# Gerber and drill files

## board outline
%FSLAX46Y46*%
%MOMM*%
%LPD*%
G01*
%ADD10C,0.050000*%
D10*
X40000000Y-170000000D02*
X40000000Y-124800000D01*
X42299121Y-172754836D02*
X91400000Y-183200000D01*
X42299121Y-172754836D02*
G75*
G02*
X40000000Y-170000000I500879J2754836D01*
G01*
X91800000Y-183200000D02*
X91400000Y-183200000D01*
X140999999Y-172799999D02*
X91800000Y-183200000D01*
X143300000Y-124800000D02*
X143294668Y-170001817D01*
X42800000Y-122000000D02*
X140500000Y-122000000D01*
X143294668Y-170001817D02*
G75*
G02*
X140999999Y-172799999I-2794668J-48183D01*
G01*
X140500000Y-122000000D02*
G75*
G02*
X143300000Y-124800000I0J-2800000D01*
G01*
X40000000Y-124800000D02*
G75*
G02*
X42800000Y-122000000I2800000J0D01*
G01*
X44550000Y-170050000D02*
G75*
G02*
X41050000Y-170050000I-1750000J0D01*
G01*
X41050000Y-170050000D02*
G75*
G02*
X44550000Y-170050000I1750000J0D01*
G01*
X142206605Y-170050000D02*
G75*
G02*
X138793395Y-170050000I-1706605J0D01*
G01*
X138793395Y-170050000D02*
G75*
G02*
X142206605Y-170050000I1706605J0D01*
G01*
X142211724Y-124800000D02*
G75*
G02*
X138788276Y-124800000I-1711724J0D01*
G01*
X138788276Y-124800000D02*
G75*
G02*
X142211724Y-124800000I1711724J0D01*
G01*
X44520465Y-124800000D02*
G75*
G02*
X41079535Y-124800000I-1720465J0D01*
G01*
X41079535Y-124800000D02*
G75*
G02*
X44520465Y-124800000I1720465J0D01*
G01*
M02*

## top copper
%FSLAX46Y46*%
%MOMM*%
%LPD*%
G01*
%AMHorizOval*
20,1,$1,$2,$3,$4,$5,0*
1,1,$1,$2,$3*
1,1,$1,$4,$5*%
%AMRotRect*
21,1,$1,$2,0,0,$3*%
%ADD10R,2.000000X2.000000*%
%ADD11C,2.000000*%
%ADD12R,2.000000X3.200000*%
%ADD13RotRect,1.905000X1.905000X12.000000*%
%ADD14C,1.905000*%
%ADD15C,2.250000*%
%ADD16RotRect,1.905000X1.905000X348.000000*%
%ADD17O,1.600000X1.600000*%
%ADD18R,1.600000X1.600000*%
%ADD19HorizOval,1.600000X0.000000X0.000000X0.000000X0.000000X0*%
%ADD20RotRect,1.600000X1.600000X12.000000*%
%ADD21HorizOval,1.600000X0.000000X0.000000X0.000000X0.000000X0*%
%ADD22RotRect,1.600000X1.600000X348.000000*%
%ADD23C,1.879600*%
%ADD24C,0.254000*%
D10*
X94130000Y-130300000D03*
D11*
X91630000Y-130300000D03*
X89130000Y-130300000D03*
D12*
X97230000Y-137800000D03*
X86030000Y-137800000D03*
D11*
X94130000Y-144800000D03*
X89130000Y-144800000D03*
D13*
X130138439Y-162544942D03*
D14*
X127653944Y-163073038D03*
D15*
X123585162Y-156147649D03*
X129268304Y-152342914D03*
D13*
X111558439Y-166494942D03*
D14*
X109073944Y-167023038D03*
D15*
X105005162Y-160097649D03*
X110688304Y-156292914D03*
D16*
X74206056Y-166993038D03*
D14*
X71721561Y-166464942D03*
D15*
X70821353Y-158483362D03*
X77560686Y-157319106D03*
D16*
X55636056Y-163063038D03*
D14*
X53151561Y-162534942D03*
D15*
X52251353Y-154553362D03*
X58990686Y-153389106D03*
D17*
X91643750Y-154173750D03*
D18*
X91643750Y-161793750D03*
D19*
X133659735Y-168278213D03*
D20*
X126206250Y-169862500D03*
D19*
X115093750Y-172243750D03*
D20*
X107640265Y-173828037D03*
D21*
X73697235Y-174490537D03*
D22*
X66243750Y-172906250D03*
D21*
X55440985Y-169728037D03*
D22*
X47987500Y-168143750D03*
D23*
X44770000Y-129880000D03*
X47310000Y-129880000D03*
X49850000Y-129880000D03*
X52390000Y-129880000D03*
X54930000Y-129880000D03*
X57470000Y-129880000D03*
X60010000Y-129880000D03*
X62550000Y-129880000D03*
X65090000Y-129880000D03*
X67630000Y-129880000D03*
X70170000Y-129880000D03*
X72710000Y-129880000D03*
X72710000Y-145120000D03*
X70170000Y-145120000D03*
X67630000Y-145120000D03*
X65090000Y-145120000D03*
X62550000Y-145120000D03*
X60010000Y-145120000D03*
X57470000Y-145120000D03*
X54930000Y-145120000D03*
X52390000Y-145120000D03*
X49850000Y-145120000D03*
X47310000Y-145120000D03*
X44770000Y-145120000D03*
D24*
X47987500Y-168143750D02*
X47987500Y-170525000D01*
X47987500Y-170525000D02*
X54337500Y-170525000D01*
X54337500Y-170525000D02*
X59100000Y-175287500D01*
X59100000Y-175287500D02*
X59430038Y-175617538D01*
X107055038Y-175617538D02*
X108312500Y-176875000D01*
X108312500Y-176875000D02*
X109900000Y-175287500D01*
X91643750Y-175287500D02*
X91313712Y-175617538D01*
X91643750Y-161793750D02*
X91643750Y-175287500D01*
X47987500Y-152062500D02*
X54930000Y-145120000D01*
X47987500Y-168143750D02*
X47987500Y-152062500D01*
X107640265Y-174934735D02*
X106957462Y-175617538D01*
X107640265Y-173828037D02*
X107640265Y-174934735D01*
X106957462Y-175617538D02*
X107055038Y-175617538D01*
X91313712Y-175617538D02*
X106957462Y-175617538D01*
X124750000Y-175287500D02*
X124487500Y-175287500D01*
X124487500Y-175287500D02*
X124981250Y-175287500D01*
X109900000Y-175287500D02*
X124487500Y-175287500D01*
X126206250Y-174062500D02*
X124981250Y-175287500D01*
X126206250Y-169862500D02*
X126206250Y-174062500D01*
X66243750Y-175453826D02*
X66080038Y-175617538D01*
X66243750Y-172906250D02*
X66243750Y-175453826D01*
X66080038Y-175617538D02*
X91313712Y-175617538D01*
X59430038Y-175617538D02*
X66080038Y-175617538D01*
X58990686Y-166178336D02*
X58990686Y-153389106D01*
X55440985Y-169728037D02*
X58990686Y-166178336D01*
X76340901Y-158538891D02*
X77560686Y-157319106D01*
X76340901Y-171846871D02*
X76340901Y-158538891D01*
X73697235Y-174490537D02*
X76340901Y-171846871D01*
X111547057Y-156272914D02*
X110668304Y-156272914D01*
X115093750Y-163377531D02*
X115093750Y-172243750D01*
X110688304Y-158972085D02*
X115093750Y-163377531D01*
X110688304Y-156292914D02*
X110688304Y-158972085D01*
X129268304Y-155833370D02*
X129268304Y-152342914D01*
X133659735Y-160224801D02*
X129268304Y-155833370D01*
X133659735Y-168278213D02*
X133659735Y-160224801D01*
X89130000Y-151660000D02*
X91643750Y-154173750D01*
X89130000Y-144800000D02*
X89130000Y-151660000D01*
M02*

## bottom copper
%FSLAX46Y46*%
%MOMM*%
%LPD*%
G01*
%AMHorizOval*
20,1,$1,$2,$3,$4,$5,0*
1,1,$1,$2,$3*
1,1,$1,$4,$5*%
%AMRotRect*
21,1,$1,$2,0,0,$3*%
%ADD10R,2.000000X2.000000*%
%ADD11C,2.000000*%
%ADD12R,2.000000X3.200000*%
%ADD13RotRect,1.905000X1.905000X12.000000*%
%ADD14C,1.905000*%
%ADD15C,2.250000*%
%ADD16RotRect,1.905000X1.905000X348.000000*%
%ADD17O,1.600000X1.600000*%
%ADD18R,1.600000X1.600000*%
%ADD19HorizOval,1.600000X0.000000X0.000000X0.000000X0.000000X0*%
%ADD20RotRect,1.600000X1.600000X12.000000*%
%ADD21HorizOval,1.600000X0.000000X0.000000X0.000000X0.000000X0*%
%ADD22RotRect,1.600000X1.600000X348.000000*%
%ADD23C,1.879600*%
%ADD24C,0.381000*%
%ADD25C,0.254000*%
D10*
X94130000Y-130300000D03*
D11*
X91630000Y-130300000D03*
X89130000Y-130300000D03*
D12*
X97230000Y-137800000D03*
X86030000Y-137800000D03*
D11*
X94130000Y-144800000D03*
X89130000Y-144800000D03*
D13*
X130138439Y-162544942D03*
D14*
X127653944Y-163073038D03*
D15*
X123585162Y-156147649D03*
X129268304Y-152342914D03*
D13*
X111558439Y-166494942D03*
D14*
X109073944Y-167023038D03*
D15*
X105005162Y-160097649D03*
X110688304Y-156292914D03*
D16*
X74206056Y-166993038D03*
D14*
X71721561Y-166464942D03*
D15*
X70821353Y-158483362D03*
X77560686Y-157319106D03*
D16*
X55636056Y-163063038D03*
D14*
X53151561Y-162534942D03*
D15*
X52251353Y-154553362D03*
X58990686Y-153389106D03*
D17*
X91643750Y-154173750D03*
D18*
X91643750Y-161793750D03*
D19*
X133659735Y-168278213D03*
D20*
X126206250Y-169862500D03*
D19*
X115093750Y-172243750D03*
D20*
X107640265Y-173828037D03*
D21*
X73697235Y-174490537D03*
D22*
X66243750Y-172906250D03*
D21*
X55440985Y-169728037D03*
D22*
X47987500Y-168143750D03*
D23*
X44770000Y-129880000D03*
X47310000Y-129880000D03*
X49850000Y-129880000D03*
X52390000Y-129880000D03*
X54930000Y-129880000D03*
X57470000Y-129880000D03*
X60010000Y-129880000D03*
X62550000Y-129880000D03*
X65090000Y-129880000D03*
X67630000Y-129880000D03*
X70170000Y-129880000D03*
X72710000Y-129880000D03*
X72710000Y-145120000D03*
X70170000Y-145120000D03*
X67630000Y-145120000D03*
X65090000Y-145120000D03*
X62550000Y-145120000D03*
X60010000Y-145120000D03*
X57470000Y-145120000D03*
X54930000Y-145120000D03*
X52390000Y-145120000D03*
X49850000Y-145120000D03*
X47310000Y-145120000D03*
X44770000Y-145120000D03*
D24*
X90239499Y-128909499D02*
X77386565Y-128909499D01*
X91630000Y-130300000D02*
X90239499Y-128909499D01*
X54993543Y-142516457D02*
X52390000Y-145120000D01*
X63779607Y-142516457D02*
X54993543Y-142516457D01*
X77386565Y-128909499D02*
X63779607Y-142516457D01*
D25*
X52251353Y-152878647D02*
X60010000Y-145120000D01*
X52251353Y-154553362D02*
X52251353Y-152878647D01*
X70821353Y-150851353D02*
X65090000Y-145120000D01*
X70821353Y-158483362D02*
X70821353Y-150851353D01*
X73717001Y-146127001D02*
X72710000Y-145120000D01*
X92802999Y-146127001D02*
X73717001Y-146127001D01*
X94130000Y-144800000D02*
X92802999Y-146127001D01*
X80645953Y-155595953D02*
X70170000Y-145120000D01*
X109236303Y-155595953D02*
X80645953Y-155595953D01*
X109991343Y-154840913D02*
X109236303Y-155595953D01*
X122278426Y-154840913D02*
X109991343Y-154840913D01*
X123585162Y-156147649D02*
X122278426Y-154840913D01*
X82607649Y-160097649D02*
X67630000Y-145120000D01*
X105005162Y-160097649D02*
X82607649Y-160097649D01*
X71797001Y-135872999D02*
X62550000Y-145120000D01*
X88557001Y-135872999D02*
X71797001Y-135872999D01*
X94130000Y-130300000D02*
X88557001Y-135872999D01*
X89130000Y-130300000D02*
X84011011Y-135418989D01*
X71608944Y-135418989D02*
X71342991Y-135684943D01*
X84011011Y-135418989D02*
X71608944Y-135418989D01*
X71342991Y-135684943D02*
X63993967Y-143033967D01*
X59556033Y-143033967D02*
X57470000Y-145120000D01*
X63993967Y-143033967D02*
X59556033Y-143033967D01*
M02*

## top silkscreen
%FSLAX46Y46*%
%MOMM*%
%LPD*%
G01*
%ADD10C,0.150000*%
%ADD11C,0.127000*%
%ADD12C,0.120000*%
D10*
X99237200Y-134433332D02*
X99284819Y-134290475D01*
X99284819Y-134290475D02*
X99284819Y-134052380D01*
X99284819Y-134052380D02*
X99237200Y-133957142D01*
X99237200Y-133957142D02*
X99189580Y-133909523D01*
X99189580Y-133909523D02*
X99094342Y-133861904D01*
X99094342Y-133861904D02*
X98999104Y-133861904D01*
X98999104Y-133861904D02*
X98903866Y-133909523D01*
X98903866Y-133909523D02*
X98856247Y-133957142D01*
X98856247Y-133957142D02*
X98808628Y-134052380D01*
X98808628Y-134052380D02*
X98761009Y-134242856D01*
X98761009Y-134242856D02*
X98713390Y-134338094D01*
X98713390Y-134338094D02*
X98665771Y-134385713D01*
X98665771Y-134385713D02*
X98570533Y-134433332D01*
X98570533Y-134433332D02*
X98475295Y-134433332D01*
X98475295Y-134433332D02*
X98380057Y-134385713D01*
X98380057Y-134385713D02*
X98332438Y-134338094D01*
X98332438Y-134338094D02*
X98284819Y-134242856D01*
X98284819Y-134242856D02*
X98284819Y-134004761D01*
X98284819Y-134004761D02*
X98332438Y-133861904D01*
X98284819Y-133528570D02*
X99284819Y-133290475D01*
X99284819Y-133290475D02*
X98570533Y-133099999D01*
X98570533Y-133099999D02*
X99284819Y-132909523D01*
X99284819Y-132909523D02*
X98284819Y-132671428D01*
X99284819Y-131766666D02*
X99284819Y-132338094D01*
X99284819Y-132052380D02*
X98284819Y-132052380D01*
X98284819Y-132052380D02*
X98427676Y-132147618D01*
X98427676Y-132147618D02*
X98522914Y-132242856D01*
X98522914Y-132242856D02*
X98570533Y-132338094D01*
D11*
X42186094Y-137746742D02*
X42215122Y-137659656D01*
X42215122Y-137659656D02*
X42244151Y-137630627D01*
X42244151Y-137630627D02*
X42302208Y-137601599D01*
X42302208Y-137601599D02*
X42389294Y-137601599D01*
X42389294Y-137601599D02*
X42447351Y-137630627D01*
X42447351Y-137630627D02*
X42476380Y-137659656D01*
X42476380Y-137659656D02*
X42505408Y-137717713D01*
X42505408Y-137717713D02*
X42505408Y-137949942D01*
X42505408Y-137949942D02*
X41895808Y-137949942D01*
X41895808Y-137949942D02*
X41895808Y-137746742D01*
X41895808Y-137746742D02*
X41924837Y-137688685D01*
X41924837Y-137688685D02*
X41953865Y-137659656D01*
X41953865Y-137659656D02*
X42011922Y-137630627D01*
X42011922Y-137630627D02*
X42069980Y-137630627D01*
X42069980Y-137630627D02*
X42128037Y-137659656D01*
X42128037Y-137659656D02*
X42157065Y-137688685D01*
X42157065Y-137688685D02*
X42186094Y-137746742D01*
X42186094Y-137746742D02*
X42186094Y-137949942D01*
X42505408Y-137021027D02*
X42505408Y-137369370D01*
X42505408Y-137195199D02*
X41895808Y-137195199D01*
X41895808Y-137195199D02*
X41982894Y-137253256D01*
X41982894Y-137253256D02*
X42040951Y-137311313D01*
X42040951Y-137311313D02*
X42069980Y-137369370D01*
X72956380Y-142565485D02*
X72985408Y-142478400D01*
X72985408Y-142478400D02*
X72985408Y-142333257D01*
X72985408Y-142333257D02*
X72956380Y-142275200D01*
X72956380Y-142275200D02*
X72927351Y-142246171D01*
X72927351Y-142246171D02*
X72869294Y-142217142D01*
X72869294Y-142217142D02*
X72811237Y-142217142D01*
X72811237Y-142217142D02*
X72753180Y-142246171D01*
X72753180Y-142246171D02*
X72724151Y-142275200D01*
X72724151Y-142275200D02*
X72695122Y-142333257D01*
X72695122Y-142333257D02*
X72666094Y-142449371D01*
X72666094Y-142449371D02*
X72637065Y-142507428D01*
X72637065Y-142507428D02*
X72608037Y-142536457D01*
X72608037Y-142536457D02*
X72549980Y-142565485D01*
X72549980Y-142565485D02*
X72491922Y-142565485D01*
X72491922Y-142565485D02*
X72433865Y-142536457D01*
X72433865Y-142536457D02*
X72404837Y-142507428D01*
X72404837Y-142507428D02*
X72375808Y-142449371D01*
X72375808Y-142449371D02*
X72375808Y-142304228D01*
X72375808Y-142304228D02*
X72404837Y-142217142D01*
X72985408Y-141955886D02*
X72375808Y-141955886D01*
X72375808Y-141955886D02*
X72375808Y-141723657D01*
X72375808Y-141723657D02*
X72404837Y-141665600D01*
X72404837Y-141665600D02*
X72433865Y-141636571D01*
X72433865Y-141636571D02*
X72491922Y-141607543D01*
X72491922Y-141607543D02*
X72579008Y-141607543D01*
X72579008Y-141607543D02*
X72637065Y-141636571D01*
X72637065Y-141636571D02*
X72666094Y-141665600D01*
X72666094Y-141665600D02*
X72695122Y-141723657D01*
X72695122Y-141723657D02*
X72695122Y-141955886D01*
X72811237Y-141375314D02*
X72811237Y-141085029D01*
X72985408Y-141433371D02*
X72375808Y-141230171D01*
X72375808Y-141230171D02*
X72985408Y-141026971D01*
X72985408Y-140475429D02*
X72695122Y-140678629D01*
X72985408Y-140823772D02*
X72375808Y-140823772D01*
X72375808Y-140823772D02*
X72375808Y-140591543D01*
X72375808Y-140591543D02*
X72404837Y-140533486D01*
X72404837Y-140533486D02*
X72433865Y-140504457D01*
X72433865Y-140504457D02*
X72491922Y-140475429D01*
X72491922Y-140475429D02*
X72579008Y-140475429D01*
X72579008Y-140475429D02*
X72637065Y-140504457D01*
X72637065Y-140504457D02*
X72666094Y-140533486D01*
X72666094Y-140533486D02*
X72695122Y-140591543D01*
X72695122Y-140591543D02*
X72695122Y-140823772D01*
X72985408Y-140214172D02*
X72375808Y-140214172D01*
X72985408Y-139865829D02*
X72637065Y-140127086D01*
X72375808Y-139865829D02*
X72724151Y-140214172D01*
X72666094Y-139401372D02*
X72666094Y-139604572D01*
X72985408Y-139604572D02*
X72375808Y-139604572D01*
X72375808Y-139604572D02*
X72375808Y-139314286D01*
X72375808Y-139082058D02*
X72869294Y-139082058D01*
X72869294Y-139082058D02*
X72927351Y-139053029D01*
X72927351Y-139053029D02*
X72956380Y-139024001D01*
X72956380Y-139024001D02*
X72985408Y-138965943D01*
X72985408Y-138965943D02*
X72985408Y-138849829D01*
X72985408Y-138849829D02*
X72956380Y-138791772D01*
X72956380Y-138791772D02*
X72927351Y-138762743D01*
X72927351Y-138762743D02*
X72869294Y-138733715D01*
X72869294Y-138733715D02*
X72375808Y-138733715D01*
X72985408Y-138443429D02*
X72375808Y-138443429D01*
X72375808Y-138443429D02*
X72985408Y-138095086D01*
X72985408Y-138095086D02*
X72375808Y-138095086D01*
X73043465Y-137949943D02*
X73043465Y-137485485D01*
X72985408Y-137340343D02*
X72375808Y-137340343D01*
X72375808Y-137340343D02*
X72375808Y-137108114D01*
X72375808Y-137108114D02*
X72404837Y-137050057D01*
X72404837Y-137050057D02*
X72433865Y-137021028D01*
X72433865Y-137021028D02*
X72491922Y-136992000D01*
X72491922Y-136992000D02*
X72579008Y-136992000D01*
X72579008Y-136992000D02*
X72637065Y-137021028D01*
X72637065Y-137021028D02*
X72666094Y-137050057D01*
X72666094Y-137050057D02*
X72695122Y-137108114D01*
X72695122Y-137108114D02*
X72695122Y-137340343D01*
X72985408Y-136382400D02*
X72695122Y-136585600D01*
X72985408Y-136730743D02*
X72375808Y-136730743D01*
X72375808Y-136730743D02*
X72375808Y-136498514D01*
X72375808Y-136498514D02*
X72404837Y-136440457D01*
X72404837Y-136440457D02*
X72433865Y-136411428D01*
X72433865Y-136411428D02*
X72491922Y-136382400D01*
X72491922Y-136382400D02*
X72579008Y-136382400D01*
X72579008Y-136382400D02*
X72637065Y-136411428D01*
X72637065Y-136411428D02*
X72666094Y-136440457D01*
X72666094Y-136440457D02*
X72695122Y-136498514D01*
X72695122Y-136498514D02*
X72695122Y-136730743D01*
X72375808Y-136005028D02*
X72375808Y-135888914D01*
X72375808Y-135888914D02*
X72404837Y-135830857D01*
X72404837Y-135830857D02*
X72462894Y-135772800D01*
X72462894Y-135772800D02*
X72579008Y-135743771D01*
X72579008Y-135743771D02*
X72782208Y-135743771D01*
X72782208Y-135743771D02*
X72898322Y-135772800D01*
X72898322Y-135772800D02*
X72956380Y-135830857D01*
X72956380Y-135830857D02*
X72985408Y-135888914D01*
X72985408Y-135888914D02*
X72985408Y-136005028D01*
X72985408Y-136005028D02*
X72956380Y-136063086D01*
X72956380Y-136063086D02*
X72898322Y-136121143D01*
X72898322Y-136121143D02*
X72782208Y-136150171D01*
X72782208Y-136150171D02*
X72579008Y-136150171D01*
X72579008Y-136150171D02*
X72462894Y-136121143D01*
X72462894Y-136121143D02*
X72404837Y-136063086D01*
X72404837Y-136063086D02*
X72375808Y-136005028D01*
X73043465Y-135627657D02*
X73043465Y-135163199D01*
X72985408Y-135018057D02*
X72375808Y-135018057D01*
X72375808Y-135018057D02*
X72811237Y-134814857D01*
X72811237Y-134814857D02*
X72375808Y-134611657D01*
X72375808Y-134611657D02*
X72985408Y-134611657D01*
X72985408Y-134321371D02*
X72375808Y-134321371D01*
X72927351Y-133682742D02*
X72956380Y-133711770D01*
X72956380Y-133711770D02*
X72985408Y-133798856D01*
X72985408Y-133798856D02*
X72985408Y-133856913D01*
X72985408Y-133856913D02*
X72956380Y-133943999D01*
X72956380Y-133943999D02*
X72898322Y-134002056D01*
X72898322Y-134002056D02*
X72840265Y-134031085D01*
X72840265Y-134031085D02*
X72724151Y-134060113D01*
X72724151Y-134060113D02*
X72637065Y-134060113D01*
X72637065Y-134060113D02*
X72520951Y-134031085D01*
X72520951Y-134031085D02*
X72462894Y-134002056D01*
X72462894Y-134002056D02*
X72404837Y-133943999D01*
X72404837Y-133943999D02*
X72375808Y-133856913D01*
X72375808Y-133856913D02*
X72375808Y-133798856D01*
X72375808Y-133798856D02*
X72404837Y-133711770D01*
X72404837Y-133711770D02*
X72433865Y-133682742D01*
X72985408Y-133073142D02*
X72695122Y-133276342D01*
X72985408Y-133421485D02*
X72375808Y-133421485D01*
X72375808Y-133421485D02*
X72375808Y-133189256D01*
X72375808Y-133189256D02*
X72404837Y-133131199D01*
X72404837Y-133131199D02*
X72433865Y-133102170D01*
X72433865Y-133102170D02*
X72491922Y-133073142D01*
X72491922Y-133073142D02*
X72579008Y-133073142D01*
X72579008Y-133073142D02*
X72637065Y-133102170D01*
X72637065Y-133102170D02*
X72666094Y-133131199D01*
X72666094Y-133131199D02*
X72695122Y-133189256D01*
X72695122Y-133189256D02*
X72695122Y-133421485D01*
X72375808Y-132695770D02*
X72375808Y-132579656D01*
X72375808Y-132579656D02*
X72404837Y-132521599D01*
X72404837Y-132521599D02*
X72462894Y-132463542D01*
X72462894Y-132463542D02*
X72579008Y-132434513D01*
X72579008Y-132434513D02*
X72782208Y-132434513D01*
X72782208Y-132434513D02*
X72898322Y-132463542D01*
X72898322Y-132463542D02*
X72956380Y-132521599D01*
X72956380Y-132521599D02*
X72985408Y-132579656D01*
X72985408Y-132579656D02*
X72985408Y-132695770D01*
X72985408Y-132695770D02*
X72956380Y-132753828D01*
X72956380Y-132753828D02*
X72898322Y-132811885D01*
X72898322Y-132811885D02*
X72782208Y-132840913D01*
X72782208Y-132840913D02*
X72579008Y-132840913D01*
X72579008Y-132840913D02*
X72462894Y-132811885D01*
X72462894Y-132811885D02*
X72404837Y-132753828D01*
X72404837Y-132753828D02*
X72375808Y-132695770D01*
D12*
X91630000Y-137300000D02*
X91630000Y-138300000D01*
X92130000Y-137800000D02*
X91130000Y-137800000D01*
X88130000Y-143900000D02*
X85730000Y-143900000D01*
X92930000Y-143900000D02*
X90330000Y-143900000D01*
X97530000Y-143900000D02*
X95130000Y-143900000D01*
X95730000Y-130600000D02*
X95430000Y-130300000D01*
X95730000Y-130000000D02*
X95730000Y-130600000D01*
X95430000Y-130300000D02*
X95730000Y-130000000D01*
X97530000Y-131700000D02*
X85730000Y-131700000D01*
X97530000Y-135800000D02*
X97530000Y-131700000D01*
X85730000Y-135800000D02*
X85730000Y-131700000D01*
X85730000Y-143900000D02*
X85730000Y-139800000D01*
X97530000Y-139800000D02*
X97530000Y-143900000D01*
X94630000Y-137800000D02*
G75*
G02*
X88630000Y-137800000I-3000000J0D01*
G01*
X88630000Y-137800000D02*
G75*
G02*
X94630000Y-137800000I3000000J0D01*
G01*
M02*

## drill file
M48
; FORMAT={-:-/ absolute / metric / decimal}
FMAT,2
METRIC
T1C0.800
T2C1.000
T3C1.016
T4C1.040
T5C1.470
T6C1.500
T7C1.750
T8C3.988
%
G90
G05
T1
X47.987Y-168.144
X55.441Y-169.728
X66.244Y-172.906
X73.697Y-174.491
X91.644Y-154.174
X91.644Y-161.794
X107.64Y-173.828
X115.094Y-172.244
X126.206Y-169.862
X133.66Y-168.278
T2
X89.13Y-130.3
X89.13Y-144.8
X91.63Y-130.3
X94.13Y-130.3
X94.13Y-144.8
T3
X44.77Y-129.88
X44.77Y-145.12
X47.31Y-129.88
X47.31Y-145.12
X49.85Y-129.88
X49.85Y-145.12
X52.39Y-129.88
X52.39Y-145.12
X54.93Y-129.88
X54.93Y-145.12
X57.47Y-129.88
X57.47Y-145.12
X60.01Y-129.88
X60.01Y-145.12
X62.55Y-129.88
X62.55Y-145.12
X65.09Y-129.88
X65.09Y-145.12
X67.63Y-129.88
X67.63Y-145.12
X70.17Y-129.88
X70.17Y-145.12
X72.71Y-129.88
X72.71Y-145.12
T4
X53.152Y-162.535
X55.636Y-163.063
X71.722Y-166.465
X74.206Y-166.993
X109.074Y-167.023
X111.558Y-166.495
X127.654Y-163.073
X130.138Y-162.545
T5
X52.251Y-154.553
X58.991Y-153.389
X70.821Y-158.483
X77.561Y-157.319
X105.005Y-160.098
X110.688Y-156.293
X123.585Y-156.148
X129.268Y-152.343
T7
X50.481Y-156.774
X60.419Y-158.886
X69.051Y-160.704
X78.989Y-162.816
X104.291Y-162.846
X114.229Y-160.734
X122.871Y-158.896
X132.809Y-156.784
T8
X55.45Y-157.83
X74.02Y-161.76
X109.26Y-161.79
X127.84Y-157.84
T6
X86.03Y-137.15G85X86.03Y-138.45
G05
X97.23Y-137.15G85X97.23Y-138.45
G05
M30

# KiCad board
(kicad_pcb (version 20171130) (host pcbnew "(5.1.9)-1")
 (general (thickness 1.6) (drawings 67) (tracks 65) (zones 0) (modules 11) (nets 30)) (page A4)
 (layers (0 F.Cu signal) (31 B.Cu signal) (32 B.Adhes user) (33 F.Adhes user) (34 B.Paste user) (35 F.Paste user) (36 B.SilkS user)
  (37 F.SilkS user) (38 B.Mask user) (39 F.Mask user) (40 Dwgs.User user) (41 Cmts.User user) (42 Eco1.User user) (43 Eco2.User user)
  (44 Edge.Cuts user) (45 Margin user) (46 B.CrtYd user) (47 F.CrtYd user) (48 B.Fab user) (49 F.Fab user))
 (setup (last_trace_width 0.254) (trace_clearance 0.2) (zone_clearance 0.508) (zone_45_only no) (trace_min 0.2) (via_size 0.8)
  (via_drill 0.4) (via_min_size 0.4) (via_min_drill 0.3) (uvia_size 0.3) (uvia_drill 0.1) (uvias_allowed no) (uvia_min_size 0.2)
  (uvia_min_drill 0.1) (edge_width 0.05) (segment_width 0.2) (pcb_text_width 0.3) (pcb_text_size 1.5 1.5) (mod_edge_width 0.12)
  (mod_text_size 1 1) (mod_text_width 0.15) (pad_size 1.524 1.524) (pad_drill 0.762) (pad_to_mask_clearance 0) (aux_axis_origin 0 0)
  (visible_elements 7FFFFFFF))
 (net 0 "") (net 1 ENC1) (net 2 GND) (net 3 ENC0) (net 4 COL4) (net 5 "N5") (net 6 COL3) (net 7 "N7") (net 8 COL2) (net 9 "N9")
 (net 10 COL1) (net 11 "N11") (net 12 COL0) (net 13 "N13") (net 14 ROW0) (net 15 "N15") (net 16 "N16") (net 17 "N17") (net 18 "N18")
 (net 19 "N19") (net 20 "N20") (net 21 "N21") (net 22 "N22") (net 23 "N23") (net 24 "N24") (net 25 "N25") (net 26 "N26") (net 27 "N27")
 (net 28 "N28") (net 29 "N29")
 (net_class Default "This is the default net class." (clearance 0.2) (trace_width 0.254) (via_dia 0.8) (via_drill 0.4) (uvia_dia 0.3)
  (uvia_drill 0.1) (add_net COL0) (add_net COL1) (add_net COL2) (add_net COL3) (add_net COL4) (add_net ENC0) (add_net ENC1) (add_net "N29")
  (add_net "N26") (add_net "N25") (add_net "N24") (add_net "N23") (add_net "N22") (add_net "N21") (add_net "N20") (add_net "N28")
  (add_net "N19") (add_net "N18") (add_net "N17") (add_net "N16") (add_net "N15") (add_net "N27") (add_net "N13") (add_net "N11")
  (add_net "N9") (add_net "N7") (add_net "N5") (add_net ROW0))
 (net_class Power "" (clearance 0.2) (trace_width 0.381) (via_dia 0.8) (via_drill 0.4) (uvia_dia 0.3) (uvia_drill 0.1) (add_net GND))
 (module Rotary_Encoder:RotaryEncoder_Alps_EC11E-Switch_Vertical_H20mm (layer F.Cu) (at 94.13 130.3 270)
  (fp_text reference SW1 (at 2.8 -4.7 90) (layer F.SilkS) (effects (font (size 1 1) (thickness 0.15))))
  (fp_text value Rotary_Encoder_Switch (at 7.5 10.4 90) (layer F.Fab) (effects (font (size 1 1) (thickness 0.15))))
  (fp_line (start 7 2.5) (end 8 2.5) (layer F.SilkS) (width 0.12))
  (fp_line (start 7.5 2) (end 7.5 3) (layer F.SilkS) (width 0.12))
  (fp_line (start 13.6 6) (end 13.6 8.4) (layer F.SilkS) (width 0.12))
  (fp_line (start 13.6 1.2) (end 13.6 3.8) (layer F.SilkS) (width 0.12))
  (fp_line (start 13.6 -3.4) (end 13.6 -1) (layer F.SilkS) (width 0.12))
  (fp_line (start 0.3 -1.6) (end 0 -1.3) (layer F.SilkS) (width 0.12))
  (fp_line (start -0.3 -1.6) (end 0.3 -1.6) (layer F.SilkS) (width 0.12))
  (fp_line (start 0 -1.3) (end -0.3 -1.6) (layer F.SilkS) (width 0.12))
  (fp_line (start 1.4 -3.4) (end 1.4 8.4) (layer F.SilkS) (width 0.12))
  (fp_line (start 5.5 -3.4) (end 1.4 -3.4) (layer F.SilkS) (width 0.12))
  (fp_line (start 5.5 8.4) (end 1.4 8.4) (layer F.SilkS) (width 0.12))
  (fp_line (start 13.6 8.4) (end 9.5 8.4) (layer F.SilkS) (width 0.12))
  (fp_line (start 9.5 -3.4) (end 13.6 -3.4) (layer F.SilkS) (width 0.12))
  (fp_circle (center 7.5 2.5) (end 10.5 2.5) (layer F.SilkS) (width 0.12))
  (pad A thru_hole rect (at 0 0 270) (size 2 2) (drill 1) (layers *.Cu *.Mask) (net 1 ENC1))
  (pad C thru_hole circle (at 0 2.5 270) (size 2 2) (drill 1) (layers *.Cu *.Mask) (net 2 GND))
  (pad B thru_hole circle (at 0 5 270) (size 2 2) (drill 1) (layers *.Cu *.Mask) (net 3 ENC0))
  (pad MP thru_hole rect (at 7.5 -3.1 270) (size 3.2 2) (drill oval 2.8 1.5) (layers *.Cu *.Mask))
  (pad MP thru_hole rect (at 7.5 8.1 270) (size 3.2 2) (drill oval 2.8 1.5) (layers *.Cu *.Mask))
  (pad S2 thru_hole circle (at 14.5 0 270) (size 2 2) (drill 1) (layers *.Cu *.Mask) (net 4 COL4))
  (pad S1 thru_hole circle (at 14.5 5 270) (size 2 2) (drill 1) (layers *.Cu *.Mask) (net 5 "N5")))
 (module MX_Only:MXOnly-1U (layer F.Cu) (at 127.84 157.84 12)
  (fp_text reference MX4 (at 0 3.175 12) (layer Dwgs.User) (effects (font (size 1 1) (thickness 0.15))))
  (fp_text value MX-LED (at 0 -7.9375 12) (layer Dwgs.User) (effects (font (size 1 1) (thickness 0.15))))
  (pad "" np_thru_hole circle (at 5.08 0 60.0996) (size 1.75 1.75) (drill 1.75) (layers *.Cu *.Mask))
  (pad "" np_thru_hole circle (at -5.08 0 60.0996) (size 1.75 1.75) (drill 1.75) (layers *.Cu *.Mask))
  (pad 4 thru_hole rect (at 1.27 5.08 12) (size 1.905 1.905) (drill 1.04) (layers *.Cu B.Mask))
  (pad 3 thru_hole circle (at -1.27 5.08 12) (size 1.905 1.905) (drill 1.04) (layers *.Cu B.Mask))
  (pad 1 thru_hole circle (at -3.81 -2.54 12) (size 2.25 2.25) (drill 1.47) (layers *.Cu B.Mask) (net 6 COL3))
  (pad "" np_thru_hole circle (at 0 0 12) (size 3.9878 3.9878) (drill 3.9878) (layers *.Cu *.Mask))
  (pad 2 thru_hole circle (at 2.54 -5.08 12) (size 2.25 2.25) (drill 1.47) (layers *.Cu B.Mask) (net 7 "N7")))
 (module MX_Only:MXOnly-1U (layer F.Cu) (at 109.26 161.79 12)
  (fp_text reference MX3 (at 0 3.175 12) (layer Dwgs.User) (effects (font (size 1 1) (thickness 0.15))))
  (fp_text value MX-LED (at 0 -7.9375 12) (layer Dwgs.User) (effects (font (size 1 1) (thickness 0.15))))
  (pad "" np_thru_hole circle (at 5.08 0 60.0996) (size 1.75 1.75) (drill 1.75) (layers *.Cu *.Mask))
  (pad "" np_thru_hole circle (at -5.08 0 60.0996) (size 1.75 1.75) (drill 1.75) (layers *.Cu *.Mask))
  (pad 4 thru_hole rect (at 1.27 5.08 12) (size 1.905 1.905) (drill 1.04) (layers *.Cu B.Mask))
  (pad 3 thru_hole circle (at -1.27 5.08 12) (size 1.905 1.905) (drill 1.04) (layers *.Cu B.Mask))
  (pad 1 thru_hole circle (at -3.81 -2.54 12) (size 2.25 2.25) (drill 1.47) (layers *.Cu B.Mask) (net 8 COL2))
  (pad "" np_thru_hole circle (at 0 0 12) (size 3.9878 3.9878) (drill 3.9878) (layers *.Cu *.Mask))
  (pad 2 thru_hole circle (at 2.54 -5.08 12) (size 2.25 2.25) (drill 1.47) (layers *.Cu B.Mask) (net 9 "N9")))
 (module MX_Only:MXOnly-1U (layer F.Cu) (at 74.02 161.76 348)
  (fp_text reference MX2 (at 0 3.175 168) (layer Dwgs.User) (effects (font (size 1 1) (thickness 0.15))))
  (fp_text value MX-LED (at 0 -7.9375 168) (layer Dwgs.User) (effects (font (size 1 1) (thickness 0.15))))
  (pad "" np_thru_hole circle (at 5.08 0 36.0996) (size 1.75 1.75) (drill 1.75) (layers *.Cu *.Mask))
  (pad "" np_thru_hole circle (at -5.08 0 36.0996) (size 1.75 1.75) (drill 1.75) (layers *.Cu *.Mask))
  (pad 4 thru_hole rect (at 1.27 5.08 348) (size 1.905 1.905) (drill 1.04) (layers *.Cu B.Mask))
  (pad 3 thru_hole circle (at -1.27 5.08 348) (size 1.905 1.905) (drill 1.04) (layers *.Cu B.Mask))
  (pad 1 thru_hole circle (at -3.81 -2.54 348) (size 2.25 2.25) (drill 1.47) (layers *.Cu B.Mask) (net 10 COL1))
  (pad "" np_thru_hole circle (at 0 0 348) (size 3.9878 3.9878) (drill 3.9878) (layers *.Cu *.Mask))
  (pad 2 thru_hole circle (at 2.54 -5.08 348) (size 2.25 2.25) (drill 1.47) (layers *.Cu B.Mask) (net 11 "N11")))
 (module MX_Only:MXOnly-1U (layer F.Cu) (at 55.45 157.83 348)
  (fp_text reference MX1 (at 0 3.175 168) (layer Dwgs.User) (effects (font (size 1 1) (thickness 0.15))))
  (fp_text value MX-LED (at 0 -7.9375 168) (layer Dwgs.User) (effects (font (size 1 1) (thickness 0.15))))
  (pad "" np_thru_hole circle (at 5.08 0 36.0996) (size 1.75 1.75) (drill 1.75) (layers *.Cu *.Mask))
  (pad "" np_thru_hole circle (at -5.08 0 36.0996) (size 1.75 1.75) (drill 1.75) (layers *.Cu *.Mask))
  (pad 4 thru_hole rect (at 1.27 5.08 348) (size 1.905 1.905) (drill 1.04) (layers *.Cu B.Mask))
  (pad 3 thru_hole circle (at -1.27 5.08 348) (size 1.905 1.905) (drill 1.04) (layers *.Cu B.Mask))
  (pad 1 thru_hole circle (at -3.81 -2.54 348) (size 2.25 2.25) (drill 1.47) (layers *.Cu B.Mask) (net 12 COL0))
  (pad "" np_thru_hole circle (at 0 0 348) (size 3.9878 3.9878) (drill 3.9878) (layers *.Cu *.Mask))
  (pad 2 thru_hole circle (at 2.54 -5.08 348) (size 2.25 2.25) (drill 1.47) (layers *.Cu B.Mask) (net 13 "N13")))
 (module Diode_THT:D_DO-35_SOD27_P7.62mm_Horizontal (layer B.Cu) (at 91.64375 161.79375 90)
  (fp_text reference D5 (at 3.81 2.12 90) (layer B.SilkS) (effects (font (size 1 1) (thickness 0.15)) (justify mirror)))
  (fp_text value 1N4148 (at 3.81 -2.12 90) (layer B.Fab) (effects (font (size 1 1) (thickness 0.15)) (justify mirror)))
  (pad 2 thru_hole oval (at 7.62 0 90) (size 1.6 1.6) (drill 0.8) (layers *.Cu *.Mask) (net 5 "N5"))
  (pad 1 thru_hole rect (at 0 0 90) (size 1.6 1.6) (drill 0.8) (layers *.Cu *.Mask) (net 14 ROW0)))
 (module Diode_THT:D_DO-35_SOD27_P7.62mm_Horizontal (layer B.Cu) (at 126.20625 169.8625 12)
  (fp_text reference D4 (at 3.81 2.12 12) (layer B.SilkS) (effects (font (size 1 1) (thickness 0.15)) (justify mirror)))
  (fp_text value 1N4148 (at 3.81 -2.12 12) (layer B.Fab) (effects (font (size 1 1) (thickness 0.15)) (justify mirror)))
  (pad 2 thru_hole oval (at 7.62 0 12) (size 1.6 1.6) (drill 0.8) (layers *.Cu *.Mask) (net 7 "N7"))
  (pad 1 thru_hole rect (at 0 0 12) (size 1.6 1.6) (drill 0.8) (layers *.Cu *.Mask) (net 14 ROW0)))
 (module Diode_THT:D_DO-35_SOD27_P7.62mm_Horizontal (layer B.Cu) (at 107.640265 173.828037 12)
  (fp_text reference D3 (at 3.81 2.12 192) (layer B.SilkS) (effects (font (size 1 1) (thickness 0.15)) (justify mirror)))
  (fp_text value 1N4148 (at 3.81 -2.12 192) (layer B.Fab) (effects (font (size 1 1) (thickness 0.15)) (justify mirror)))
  (pad 2 thru_hole oval (at 7.62 0 12) (size 1.6 1.6) (drill 0.8) (layers *.Cu *.Mask) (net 9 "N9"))
  (pad 1 thru_hole rect (at 0 0 12) (size 1.6 1.6) (drill 0.8) (layers *.Cu *.Mask) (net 14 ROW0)))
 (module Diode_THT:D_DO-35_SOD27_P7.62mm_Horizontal (layer B.Cu) (at 66.24375 172.90625 348)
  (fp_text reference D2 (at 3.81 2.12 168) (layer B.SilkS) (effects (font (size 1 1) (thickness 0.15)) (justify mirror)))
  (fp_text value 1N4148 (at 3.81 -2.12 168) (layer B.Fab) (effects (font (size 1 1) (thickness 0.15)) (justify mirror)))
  (pad 2 thru_hole oval (at 7.62 0 348) (size 1.6 1.6) (drill 0.8) (layers *.Cu *.Mask) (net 11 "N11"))
  (pad 1 thru_hole rect (at 0 0 348) (size 1.6 1.6) (drill 0.8) (layers *.Cu *.Mask) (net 14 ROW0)))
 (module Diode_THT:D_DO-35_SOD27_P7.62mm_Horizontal (layer B.Cu) (at 47.9875 168.14375 348)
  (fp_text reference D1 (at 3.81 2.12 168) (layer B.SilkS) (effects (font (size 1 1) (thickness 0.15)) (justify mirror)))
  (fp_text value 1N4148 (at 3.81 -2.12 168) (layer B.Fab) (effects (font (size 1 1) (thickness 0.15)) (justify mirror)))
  (pad 2 thru_hole oval (at 7.62 0 348) (size 1.6 1.6) (drill 0.8) (layers *.Cu *.Mask) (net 13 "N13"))
  (pad 1 thru_hole rect (at 0 0 348) (size 1.6 1.6) (drill 0.8) (layers *.Cu *.Mask) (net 14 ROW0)))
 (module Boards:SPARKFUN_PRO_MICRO (layer F.Cu) (at 57.47 137.5 90)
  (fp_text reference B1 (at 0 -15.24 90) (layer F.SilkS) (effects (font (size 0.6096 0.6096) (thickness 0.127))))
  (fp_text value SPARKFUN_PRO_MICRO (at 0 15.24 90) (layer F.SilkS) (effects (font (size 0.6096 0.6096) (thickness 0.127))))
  (pad 24 thru_hole circle (at 7.62 -12.7 90) (size 1.8796 1.8796) (drill 1.016) (layers *.Cu *.Mask) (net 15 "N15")
   (solder_mask_margin 0.1016))
  (pad 23 thru_hole circle (at 7.62 -10.16 90) (size 1.8796 1.8796) (drill 1.016) (layers *.Cu *.Mask) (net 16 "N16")
   (solder_mask_margin 0.1016))
  (pad 22 thru_hole circle (at 7.62 -7.62 90) (size 1.8796 1.8796) (drill 1.016) (layers *.Cu *.Mask) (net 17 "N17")
   (solder_mask_margin 0.1016))
  (pad 21 thru_hole circle (at 7.62 -5.08 90) (size 1.8796 1.8796) (drill 1.016) (layers *.Cu *.Mask) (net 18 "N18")
   (solder_mask_margin 0.1016))
  (pad 20 thru_hole circle (at 7.62 -2.54 90) (size 1.8796 1.8796) (drill 1.016) (layers *.Cu *.Mask) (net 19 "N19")
   (solder_mask_margin 0.1016))
  (pad 19 thru_hole circle (at 7.62 0 90) (size 1.8796 1.8796) (drill 1.016) (layers *.Cu *.Mask) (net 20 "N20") (solder_mask_margin 0.1016))
  (pad 18 thru_hole circle (at 7.62 2.54 90) (size 1.8796 1.8796) (drill 1.016) (layers *.Cu *.Mask) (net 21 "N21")
   (solder_mask_margin 0.1016))
  (pad 17 thru_hole circle (at 7.62 5.08 90) (size 1.8796 1.8796) (drill 1.016) (layers *.Cu *.Mask) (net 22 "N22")
   (solder_mask_margin 0.1016))
  (pad 16 thru_hole circle (at 7.62 7.62 90) (size 1.8796 1.8796) (drill 1.016) (layers *.Cu *.Mask) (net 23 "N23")
   (solder_mask_margin 0.1016))
  (pad 15 thru_hole circle (at 7.62 10.16 90) (size 1.8796 1.8796) (drill 1.016) (layers *.Cu *.Mask) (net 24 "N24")
   (solder_mask_margin 0.1016))
  (pad 14 thru_hole circle (at 7.62 12.7 90) (size 1.8796 1.8796) (drill 1.016) (layers *.Cu *.Mask) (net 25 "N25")
   (solder_mask_margin 0.1016))
  (pad 13 thru_hole circle (at 7.62 15.24 90) (size 1.8796 1.8796) (drill 1.016) (layers *.Cu *.Mask) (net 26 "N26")
   (solder_mask_margin 0.1016))
  (pad 12 thru_hole circle (at -7.62 15.24 90) (size 1.8796 1.8796) (drill 1.016) (layers *.Cu *.Mask) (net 4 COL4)
   (solder_mask_margin 0.1016))
  (pad 11 thru_hole circle (at -7.62 12.7 90) (size 1.8796 1.8796) (drill 1.016) (layers *.Cu *.Mask) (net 6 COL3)
   (solder_mask_margin 0.1016))
  (pad 10 thru_hole circle (at -7.62 10.16 90) (size 1.8796 1.8796) (drill 1.016) (layers *.Cu *.Mask) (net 8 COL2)
   (solder_mask_margin 0.1016))
  (pad 9 thru_hole circle (at -7.62 7.62 90) (size 1.8796 1.8796) (drill 1.016) (layers *.Cu *.Mask) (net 10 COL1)
   (solder_mask_margin 0.1016))
  (pad 8 thru_hole circle (at -7.62 5.08 90) (size 1.8796 1.8796) (drill 1.016) (layers *.Cu *.Mask) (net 1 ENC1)
   (solder_mask_margin 0.1016))
  (pad 7 thru_hole circle (at -7.62 2.54 90) (size 1.8796 1.8796) (drill 1.016) (layers *.Cu *.Mask) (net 12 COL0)
   (solder_mask_margin 0.1016))
  (pad 6 thru_hole circle (at -7.62 0 90) (size 1.8796 1.8796) (drill 1.016) (layers *.Cu *.Mask) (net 3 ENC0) (solder_mask_margin 0.1016))
  (pad 5 thru_hole circle (at -7.62 -2.54 90) (size 1.8796 1.8796) (drill 1.016) (layers *.Cu *.Mask) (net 14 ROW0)
   (solder_mask_margin 0.1016))
  (pad 4 thru_hole circle (at -7.62 -5.08 90) (size 1.8796 1.8796) (drill 1.016) (layers *.Cu *.Mask) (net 2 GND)
   (solder_mask_margin 0.1016))
  (pad 3 thru_hole circle (at -7.62 -7.62 90) (size 1.8796 1.8796) (drill 1.016) (layers *.Cu *.Mask) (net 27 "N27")
   (solder_mask_margin 0.1016))
  (pad 2 thru_hole circle (at -7.62 -10.16 90) (size 1.8796 1.8796) (drill 1.016) (layers *.Cu *.Mask) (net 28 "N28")
   (solder_mask_margin 0.1016))
  (pad 1 thru_hole circle (at -7.62 -12.7 90) (size 1.8796 1.8796) (drill 1.016) (layers *.Cu *.Mask) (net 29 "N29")
   (solder_mask_margin 0.1016)))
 (gr_line (start 40 170) (end 40 124.8) (layer Edge.Cuts) (width 0.05))
 (gr_line (start 42.299121 172.754836) (end 91.4 183.2) (layer Edge.Cuts) (width 0.05))
 (gr_arc (start 42.8 170) (end 40 170) (angle -79.69515353) (layer Edge.Cuts) (width 0.05))
 (gr_line (start 91.8 183.2) (end 91.4 183.2) (layer Edge.Cuts) (width 0.05))
 (gr_line (start 140.999999 172.799999) (end 91.8 183.2) (layer Edge.Cuts) (width 0.05))
 (gr_line (start 143.3 124.8) (end 143.294668 170.001817) (layer Edge.Cuts) (width 0.05))
 (gr_line (start 42.8 122) (end 140.5 122) (layer Edge.Cuts) (width 0.05))
 (gr_arc (start 140.5 170.05) (end 140.999999 172.799999) (angle -80.68291393) (layer Edge.Cuts) (width 0.05))
 (gr_arc (start 140.5 124.8) (end 143.3 124.8) (angle -90) (layer Edge.Cuts) (width 0.05))
 (gr_arc (start 42.8 124.8) (end 42.8 122) (angle -90) (layer Edge.Cuts) (width 0.05))
 (gr_circle (center 42.8 170.05) (end 42.8 171.8) (layer Edge.Cuts) (width 0.05))
 (gr_circle (center 140.5 170.05) (end 141.95 170.95) (layer Edge.Cuts) (width 0.05))
 (gr_circle (center 140.5 124.8) (end 142.2 124.6) (layer Edge.Cuts) (width 0.05))
 (gr_circle (center 42.8 124.8) (end 41.4 123.8) (layer Edge.Cuts) (width 0.05))
 (segment (start 90.239499 128.909499) (end 77.386565 128.909499) (width 0.381) (layer B.Cu) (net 2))
 (segment (start 91.63 130.3) (end 90.239499 128.909499) (width 0.381) (layer B.Cu) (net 2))
 (segment (start 54.993543 142.516457) (end 52.39 145.12) (width 0.381) (layer B.Cu) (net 2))
 (segment (start 63.779607 142.516457) (end 54.993543 142.516457) (width 0.381) (layer B.Cu) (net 2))
 (segment (start 77.386565 128.909499) (end 63.779607 142.516457) (width 0.381) (layer B.Cu) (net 2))
 (segment (start 47.9875 168.14375) (end 47.9875 170.525) (width 0.254) (layer F.Cu) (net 14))
 (segment (start 47.9875 170.525) (end 54.3375 170.525) (width 0.254) (layer F.Cu) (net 14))
 (segment (start 54.3375 170.525) (end 59.1 175.2875) (width 0.254) (layer F.Cu) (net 14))
 (segment (start 59.1 175.2875) (end 59.430038 175.617538) (width 0.254) (layer F.Cu) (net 14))
 (segment (start 107.055038 175.617538) (end 108.3125 176.875) (width 0.254) (layer F.Cu) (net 14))
 (segment (start 108.3125 176.875) (end 109.9 175.2875) (width 0.254) (layer F.Cu) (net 14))
 (segment (start 91.64375 175.2875) (end 91.313712 175.617538) (width 0.254) (layer F.Cu) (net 14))
 (segment (start 91.64375 161.79375) (end 91.64375 175.2875) (width 0.254) (layer F.Cu) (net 14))
 (segment (start 47.9875 152.0625) (end 54.93 145.12) (width 0.254) (layer F.Cu) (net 14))
 (segment (start 47.9875 168.14375) (end 47.9875 152.0625) (width 0.254) (layer F.Cu) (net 14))
 (segment (start 107.640265 174.934735) (end 106.957462 175.617538) (width 0.254) (layer F.Cu) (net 14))
 (segment (start 107.640265 173.828037) (end 107.640265 174.934735) (width 0.254) (layer F.Cu) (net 14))
 (segment (start 106.957462 175.617538) (end 107.055038 175.617538) (width 0.254) (layer F.Cu) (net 14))
 (segment (start 91.313712 175.617538) (end 106.957462 175.617538) (width 0.254) (layer F.Cu) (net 14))
 (segment (start 124.75 175.2875) (end 124.4875 175.2875) (width 0.254) (layer F.Cu) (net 14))
 (segment (start 124.4875 175.2875) (end 124.98125 175.2875) (width 0.254) (layer F.Cu) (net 14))
 (segment (start 109.9 175.2875) (end 124.4875 175.2875) (width 0.254) (layer F.Cu) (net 14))
 (segment (start 126.20625 174.0625) (end 124.98125 175.2875) (width 0.254) (layer F.Cu) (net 14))
 (segment (start 126.20625 169.8625) (end 126.20625 174.0625) (width 0.254) (layer F.Cu) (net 14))
 (segment (start 66.24375 175.453826) (end 66.080038 175.617538) (width 0.254) (layer F.Cu) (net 14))
 (segment (start 66.24375 172.90625) (end 66.24375 175.453826) (width 0.254) (layer F.Cu) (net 14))
 (segment (start 66.080038 175.617538) (end 91.313712 175.617538) (width 0.254) (layer F.Cu) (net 14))
 (segment (start 59.430038 175.617538) (end 66.080038 175.617538) (width 0.254) (layer F.Cu) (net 14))
 (segment (start 52.251353 152.878647) (end 60.01 145.12) (width 0.254) (layer B.Cu) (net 12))
 (segment (start 52.251353 154.553362) (end 52.251353 152.878647) (width 0.254) (layer B.Cu) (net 12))
 (segment (start 70.821353 150.851353) (end 65.09 145.12) (width 0.254) (layer B.Cu) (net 10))
 (segment (start 70.821353 158.483362) (end 70.821353 150.851353) (width 0.254) (layer B.Cu) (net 10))
 (segment (start 73.717001 146.127001) (end 72.71 145.12) (width 0.254) (layer B.Cu) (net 4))
 (segment (start 92.802999 146.127001) (end 73.717001 146.127001) (width 0.254) (layer B.Cu) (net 4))
 (segment (start 94.13 144.8) (end 92.802999 146.127001) (width 0.254) (layer B.Cu) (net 4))
 (segment (start 80.645953 155.595953) (end 70.17 145.12) (width 0.254) (layer B.Cu) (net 6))
 (segment (start 109.236303 155.595953) (end 80.645953 155.595953) (width 0.254) (layer B.Cu) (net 6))
 (segment (start 109.991343 154.840913) (end 109.236303 155.595953) (width 0.254) (layer B.Cu) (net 6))
 (segment (start 122.278426 154.840913) (end 109.991343 154.840913) (width 0.254) (layer B.Cu) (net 6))
 (segment (start 123.585162 156.147649) (end 122.278426 154.840913) (width 0.254) (layer B.Cu) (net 6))
 (segment (start 82.607649 160.097649) (end 67.63 145.12) (width 0.254) (layer B.Cu) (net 8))
 (segment (start 105.005162 160.097649) (end 82.607649 160.097649) (width 0.254) (layer B.Cu) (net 8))
 (segment (start 71.797001 135.872999) (end 62.55 145.12) (width 0.254) (layer B.Cu) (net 1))
 (segment (start 88.557001 135.872999) (end 71.797001 135.872999) (width 0.254) (layer B.Cu) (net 1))
 (segment (start 94.13 130.3) (end 88.557001 135.872999) (width 0.254) (layer B.Cu) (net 1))
 (segment (start 89.13 130.3) (end 84.011011 135.418989) (width 0.254) (layer B.Cu) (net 3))
 (segment (start 71.608944 135.418989) (end 71.342991 135.684943) (width 0.254) (layer B.Cu) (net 3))
 (segment (start 84.011011 135.418989) (end 71.608944 135.418989) (width 0.254) (layer B.Cu) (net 3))
 (segment (start 71.342991 135.684943) (end 63.993967 143.033967) (width 0.254) (layer B.Cu) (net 3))
 (segment (start 59.556033 143.033967) (end 57.47 145.12) (width 0.254) (layer B.Cu) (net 3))
 (segment (start 63.993967 143.033967) (end 59.556033 143.033967) (width 0.254) (layer B.Cu) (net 3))
 (segment (start 58.990686 166.178336) (end 58.990686 153.389106) (width 0.254) (layer F.Cu) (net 13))
 (segment (start 55.440985 169.728037) (end 58.990686 166.178336) (width 0.254) (layer F.Cu) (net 13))
 (segment (start 76.340901 158.538891) (end 77.560686 157.319106) (width 0.254) (layer F.Cu) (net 11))
 (segment (start 76.340901 171.846871) (end 76.340901 158.538891) (width 0.254) (layer F.Cu) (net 11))
 (segment (start 73.697235 174.490537) (end 76.340901 171.846871) (width 0.254) (layer F.Cu) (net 11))
 (segment (start 111.547057 156.272914) (end 110.668304 156.272914) (width 0.254) (layer F.Cu) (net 9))
 (segment (start 115.09375 163.377531) (end 115.09375 172.24375) (width 0.254) (layer F.Cu) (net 9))
 (segment (start 110.688304 158.972085) (end 115.09375 163.377531) (width 0.254) (layer F.Cu) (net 9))
 (segment (start 110.688304 156.292914) (end 110.688304 158.972085) (width 0.254) (layer F.Cu) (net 9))
 (segment (start 129.268304 155.83337) (end 129.268304 152.342914) (width 0.254) (layer F.Cu) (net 7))
 (segment (start 133.659735 160.224801) (end 129.268304 155.83337) (width 0.254) (layer F.Cu) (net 7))
 (segment (start 133.659735 168.278213) (end 133.659735 160.224801) (width 0.254) (layer F.Cu) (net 7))
 (segment (start 89.13 151.66) (end 91.64375 154.17375) (width 0.254) (layer F.Cu) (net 5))
 (segment (start 89.13 144.8) (end 89.13 151.66) (width 0.254) (layer F.Cu) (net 5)))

